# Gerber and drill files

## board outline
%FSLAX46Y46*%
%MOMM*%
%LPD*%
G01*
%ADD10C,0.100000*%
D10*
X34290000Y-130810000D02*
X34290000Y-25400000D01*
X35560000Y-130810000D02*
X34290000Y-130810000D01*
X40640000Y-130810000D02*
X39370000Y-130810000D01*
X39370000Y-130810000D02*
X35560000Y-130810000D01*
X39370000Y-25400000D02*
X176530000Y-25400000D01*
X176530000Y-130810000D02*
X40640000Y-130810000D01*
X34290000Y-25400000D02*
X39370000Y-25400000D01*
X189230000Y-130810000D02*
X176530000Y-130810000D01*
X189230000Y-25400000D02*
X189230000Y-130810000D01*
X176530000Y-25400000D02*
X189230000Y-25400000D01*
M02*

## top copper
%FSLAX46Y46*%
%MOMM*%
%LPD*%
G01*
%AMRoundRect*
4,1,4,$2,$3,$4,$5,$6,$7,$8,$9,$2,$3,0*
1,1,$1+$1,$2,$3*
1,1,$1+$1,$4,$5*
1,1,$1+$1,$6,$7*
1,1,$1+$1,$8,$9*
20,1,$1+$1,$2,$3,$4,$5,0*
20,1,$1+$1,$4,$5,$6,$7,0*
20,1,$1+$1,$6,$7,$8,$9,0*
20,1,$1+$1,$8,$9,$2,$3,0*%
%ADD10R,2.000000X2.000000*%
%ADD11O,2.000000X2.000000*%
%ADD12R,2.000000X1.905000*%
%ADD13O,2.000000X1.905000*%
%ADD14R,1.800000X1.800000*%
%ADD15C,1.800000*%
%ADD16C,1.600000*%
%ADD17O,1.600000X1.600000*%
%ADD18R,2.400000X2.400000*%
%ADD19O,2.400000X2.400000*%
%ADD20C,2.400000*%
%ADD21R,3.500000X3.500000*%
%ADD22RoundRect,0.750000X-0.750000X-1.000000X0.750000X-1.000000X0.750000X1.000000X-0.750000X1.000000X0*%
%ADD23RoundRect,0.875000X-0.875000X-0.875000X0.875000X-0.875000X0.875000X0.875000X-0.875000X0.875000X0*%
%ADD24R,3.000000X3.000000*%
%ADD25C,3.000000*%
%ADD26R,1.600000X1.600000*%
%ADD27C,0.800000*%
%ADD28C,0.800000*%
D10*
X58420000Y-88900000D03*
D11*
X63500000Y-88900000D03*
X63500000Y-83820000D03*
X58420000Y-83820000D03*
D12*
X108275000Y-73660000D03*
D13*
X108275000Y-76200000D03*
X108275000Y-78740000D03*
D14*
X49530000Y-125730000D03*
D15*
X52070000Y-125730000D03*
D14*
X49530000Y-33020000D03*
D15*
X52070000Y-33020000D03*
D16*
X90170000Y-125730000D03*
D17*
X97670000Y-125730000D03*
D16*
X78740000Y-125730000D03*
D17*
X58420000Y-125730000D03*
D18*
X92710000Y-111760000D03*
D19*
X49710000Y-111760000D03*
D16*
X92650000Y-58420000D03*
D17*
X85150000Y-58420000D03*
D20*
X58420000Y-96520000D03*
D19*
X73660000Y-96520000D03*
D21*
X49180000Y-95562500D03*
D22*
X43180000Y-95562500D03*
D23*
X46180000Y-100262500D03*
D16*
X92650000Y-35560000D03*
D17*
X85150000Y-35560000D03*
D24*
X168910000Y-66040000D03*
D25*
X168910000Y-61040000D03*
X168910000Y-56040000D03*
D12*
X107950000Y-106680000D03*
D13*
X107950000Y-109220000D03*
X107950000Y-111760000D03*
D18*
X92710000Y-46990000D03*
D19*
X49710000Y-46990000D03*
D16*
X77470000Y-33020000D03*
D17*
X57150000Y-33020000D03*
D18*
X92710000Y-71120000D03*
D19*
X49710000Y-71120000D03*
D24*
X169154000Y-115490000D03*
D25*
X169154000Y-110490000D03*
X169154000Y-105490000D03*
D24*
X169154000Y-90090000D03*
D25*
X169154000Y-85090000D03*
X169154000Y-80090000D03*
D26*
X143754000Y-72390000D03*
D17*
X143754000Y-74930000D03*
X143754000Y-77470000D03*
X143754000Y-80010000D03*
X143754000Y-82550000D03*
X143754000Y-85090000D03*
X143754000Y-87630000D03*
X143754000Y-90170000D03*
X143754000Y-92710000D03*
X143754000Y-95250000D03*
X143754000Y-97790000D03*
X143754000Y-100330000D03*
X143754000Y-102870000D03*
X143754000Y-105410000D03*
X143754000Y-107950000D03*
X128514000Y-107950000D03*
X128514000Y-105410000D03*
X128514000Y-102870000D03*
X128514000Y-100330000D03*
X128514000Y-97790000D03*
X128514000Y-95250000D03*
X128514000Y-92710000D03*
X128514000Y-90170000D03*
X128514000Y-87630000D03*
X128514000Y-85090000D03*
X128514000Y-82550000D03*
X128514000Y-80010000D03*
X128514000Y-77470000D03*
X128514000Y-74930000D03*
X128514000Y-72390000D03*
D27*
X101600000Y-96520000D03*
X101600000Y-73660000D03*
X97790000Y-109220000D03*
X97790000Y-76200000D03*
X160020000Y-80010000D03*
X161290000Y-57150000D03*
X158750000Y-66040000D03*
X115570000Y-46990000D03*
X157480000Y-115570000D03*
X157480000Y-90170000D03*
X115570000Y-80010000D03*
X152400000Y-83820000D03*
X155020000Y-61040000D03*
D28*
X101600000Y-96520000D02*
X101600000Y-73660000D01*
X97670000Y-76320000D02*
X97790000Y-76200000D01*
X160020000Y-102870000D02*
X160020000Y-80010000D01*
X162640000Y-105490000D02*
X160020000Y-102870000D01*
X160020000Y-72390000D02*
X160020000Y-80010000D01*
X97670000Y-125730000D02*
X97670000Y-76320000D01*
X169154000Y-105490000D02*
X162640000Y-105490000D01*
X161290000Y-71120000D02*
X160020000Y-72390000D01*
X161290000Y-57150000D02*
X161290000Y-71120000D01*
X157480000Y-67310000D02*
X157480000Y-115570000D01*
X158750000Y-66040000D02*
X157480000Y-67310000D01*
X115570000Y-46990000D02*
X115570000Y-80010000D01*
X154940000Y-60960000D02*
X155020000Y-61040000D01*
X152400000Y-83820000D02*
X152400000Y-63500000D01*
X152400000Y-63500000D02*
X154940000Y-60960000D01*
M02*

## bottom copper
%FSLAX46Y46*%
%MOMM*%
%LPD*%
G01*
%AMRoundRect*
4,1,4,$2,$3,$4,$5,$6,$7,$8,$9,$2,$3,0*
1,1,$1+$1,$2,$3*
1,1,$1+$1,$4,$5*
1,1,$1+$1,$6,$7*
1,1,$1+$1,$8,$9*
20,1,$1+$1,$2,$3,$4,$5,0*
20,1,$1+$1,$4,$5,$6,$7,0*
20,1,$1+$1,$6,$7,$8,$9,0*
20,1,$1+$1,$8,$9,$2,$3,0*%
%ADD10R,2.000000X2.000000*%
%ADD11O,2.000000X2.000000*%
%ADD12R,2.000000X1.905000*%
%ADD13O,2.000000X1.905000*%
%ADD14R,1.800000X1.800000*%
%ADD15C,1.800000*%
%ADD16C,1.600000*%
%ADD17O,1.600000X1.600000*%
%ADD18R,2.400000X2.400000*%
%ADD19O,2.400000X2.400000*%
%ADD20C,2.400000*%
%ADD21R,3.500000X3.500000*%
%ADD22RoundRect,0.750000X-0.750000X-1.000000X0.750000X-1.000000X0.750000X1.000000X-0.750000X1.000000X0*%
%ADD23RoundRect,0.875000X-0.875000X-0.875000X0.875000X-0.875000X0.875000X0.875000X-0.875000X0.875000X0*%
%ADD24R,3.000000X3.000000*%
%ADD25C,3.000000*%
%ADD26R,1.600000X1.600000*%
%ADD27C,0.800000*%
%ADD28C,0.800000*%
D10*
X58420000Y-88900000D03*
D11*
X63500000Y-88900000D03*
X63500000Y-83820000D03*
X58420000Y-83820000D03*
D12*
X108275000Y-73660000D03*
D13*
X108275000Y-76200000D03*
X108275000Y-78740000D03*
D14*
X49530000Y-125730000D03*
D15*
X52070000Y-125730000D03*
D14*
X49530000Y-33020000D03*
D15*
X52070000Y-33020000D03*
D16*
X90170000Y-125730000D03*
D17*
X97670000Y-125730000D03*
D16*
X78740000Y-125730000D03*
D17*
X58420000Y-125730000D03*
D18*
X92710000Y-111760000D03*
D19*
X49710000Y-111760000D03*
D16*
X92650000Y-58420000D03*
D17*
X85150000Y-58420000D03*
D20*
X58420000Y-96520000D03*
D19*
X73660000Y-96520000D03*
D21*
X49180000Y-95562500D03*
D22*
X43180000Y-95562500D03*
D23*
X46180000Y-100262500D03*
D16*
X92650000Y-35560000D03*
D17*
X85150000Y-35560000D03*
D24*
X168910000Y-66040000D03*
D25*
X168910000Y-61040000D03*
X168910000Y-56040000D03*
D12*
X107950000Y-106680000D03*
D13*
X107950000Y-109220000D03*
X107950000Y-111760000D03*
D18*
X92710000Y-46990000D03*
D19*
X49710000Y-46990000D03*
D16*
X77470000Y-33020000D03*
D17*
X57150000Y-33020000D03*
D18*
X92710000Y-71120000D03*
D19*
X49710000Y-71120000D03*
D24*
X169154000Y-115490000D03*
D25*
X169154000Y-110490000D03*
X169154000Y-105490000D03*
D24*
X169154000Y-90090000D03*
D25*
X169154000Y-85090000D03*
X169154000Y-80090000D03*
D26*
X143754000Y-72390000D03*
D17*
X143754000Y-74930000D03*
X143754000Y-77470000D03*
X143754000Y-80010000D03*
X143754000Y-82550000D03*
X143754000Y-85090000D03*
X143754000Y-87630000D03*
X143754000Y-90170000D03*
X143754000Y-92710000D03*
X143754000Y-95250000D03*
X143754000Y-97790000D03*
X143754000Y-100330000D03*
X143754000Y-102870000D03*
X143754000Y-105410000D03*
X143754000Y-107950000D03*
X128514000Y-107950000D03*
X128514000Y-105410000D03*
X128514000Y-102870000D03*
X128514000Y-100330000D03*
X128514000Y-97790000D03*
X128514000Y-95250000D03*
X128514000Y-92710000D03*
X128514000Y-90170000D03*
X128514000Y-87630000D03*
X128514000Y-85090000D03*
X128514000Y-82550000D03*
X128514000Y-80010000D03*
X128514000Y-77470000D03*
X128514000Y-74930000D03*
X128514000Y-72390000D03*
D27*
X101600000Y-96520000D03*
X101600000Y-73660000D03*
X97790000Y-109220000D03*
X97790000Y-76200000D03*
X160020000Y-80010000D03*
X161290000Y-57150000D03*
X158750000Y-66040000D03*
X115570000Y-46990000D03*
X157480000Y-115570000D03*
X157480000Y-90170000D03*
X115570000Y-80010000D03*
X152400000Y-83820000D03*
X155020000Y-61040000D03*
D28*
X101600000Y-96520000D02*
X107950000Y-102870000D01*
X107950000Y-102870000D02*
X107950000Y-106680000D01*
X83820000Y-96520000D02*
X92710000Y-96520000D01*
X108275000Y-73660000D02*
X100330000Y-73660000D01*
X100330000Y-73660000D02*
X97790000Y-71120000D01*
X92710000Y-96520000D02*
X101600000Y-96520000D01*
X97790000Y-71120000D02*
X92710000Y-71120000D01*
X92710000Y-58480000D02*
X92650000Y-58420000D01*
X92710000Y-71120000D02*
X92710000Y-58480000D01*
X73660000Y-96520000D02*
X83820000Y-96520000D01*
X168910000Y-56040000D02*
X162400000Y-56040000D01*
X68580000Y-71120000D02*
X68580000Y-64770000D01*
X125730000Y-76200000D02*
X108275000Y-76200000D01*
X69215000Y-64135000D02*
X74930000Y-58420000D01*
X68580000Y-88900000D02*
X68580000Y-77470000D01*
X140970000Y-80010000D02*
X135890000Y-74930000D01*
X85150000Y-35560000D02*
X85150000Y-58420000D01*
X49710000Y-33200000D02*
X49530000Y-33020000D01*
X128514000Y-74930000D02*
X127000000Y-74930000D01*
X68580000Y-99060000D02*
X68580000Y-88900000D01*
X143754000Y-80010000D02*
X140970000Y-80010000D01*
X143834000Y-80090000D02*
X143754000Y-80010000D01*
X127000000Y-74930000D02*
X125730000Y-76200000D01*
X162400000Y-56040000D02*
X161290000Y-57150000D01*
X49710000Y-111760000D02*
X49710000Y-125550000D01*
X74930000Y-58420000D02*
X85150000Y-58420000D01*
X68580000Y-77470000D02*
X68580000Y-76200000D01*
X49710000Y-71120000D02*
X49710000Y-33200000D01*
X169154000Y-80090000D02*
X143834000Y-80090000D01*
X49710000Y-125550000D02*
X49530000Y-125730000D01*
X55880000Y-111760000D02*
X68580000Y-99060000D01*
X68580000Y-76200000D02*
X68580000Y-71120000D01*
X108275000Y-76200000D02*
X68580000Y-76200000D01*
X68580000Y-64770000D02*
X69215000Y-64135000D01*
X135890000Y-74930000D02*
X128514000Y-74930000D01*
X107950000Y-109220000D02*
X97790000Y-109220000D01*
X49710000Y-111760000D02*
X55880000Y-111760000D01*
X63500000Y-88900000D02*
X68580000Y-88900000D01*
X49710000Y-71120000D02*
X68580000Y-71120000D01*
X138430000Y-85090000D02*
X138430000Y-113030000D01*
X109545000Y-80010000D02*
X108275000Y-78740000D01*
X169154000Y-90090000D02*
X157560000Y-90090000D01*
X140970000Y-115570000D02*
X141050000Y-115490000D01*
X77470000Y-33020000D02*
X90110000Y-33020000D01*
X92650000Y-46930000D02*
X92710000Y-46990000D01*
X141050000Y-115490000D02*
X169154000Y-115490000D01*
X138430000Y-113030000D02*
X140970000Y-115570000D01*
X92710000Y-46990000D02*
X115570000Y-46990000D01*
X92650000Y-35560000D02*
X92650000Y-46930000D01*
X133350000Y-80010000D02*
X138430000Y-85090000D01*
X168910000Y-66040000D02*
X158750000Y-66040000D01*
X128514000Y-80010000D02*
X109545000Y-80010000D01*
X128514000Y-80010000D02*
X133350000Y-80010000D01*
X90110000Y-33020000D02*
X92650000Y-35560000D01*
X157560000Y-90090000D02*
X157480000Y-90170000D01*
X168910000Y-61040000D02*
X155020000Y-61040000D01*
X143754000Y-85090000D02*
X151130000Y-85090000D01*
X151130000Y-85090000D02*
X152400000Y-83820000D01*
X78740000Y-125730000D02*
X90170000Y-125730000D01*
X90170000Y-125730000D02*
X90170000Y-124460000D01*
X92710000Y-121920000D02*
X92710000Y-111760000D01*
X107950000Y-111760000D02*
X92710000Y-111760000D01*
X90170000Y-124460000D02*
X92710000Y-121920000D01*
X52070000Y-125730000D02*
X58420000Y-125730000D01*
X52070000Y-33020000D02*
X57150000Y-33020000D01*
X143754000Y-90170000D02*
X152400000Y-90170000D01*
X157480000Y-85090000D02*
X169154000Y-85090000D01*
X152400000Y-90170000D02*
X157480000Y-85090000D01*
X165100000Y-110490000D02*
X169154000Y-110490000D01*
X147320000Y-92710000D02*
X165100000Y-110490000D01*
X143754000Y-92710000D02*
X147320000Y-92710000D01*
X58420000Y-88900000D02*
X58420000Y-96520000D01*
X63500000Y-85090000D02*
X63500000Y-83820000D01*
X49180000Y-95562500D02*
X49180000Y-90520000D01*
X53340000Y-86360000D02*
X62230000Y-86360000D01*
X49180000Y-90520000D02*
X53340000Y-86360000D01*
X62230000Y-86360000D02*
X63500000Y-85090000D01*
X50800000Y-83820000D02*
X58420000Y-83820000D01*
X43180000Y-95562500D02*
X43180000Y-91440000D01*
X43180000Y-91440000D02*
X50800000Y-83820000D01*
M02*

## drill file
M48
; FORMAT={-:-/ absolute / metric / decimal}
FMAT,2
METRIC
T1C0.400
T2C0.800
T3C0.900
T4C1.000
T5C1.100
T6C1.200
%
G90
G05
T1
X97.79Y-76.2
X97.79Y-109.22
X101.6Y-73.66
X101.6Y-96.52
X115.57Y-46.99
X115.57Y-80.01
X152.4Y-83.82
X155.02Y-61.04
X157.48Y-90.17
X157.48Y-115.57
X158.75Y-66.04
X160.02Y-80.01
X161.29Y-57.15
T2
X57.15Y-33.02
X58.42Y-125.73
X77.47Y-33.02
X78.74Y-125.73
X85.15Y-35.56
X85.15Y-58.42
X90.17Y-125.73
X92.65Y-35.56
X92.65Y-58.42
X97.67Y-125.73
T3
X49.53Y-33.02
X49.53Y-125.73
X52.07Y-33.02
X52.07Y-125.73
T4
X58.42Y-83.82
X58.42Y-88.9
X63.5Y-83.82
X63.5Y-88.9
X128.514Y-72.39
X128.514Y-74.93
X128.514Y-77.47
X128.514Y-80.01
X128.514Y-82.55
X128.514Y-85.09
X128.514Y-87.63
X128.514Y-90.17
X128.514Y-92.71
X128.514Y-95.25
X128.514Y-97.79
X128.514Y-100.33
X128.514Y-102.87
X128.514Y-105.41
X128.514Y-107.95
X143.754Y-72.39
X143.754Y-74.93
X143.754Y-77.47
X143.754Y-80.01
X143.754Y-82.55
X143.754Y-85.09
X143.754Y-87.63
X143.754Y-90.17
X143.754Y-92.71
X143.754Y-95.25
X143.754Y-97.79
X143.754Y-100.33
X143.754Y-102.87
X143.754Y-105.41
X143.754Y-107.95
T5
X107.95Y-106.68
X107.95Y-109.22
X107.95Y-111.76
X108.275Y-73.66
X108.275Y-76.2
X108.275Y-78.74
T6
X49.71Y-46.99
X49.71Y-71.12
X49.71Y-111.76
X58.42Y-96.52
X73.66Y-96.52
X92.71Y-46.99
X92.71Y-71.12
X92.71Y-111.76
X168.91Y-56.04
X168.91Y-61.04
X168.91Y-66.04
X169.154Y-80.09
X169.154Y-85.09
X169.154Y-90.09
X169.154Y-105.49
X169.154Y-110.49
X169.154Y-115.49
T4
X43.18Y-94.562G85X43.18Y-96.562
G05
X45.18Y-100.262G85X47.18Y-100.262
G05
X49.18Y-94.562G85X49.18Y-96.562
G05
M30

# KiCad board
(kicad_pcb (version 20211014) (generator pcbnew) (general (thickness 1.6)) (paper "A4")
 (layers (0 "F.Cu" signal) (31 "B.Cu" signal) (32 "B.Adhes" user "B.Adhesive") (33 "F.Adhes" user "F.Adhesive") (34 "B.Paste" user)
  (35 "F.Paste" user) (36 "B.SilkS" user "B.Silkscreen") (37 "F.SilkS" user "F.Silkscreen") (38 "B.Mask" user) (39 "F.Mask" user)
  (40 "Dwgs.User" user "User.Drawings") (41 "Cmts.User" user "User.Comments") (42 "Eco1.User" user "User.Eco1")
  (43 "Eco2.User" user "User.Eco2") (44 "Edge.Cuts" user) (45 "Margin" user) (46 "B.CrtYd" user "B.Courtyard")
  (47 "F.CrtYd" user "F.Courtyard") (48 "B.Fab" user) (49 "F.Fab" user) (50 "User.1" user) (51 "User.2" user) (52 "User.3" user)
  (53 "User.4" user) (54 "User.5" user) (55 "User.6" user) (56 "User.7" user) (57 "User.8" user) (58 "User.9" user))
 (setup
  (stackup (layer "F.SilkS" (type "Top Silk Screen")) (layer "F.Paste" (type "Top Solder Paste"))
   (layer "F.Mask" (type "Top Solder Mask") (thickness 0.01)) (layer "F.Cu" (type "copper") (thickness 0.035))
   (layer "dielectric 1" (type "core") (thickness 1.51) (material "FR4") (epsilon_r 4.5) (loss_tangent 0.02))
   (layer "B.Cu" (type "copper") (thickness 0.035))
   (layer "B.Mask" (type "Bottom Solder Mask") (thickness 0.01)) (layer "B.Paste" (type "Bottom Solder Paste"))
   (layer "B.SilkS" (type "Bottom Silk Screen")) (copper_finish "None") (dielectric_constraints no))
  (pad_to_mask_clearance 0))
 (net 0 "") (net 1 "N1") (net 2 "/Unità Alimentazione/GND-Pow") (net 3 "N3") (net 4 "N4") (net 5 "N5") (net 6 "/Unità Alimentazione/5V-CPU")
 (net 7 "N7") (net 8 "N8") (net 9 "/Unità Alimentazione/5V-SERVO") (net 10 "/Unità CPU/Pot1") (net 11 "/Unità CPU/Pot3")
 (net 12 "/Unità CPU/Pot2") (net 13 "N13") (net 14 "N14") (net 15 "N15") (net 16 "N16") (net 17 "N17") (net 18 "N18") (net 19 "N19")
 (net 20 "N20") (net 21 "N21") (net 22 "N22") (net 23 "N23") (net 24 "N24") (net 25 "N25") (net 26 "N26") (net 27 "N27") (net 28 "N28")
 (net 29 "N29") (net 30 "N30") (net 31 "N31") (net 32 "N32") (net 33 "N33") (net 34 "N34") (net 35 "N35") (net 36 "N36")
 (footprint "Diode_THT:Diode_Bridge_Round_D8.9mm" (layer "F.Cu") (at 58.42 88.9 90)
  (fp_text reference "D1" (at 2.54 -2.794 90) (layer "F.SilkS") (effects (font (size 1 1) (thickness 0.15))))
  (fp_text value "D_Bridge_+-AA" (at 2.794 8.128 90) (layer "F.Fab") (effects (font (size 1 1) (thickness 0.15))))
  (pad "1" thru_hole rect (at 0 0 90) (size 2 2) (drill 1) (layers *.Cu *.Mask) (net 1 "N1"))
  (pad "2" thru_hole oval (at 0 5.08 90) (size 2 2) (drill 1) (layers *.Cu *.Mask) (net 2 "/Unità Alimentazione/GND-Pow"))
  (pad "3" thru_hole oval (at 5.08 5.08 90) (size 2 2) (drill 1) (layers *.Cu *.Mask) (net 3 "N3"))
  (pad "4" thru_hole oval (at 5.08 0 90) (size 2 2) (drill 1) (layers *.Cu *.Mask) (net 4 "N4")))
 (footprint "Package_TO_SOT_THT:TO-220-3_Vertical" (layer "F.Cu") (at 108.275 73.66 -90)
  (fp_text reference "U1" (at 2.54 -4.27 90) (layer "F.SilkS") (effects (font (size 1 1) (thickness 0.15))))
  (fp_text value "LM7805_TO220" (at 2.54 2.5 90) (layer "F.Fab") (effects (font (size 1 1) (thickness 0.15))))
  (pad "1" thru_hole rect (at 0 0 270) (size 1.905 2) (drill 1.1) (layers *.Cu *.Mask) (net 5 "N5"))
  (pad "2" thru_hole oval (at 2.54 0 270) (size 1.905 2) (drill 1.1) (layers *.Cu *.Mask) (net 2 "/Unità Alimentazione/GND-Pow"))
  (pad "3" thru_hole oval (at 5.08 0 270) (size 1.905 2) (drill 1.1) (layers *.Cu *.Mask) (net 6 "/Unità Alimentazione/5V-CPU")))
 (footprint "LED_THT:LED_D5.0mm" (layer "F.Cu") (at 49.53 125.73)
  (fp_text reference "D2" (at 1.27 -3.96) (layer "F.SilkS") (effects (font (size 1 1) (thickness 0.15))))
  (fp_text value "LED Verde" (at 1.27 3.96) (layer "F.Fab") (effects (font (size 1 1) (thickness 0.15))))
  (pad "1" thru_hole rect (at 0 0) (size 1.8 1.8) (drill 0.9) (layers *.Cu *.Mask) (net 2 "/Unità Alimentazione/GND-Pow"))
  (pad "2" thru_hole circle (at 2.54 0) (size 1.8 1.8) (drill 0.9) (layers *.Cu *.Mask) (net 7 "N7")))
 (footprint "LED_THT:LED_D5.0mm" (layer "F.Cu") (at 49.53 33.02)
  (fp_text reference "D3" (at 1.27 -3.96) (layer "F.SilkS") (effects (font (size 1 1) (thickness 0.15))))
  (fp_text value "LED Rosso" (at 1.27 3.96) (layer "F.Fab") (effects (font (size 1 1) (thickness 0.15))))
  (pad "1" thru_hole rect (at 0 0) (size 1.8 1.8) (drill 0.9) (layers *.Cu *.Mask) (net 2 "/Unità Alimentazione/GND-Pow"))
  (pad "2" thru_hole circle (at 2.54 0) (size 1.8 1.8) (drill 0.9) (layers *.Cu *.Mask) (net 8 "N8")))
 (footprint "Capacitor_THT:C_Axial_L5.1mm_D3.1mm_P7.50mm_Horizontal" (layer "F.Cu") (at 90.17 125.73)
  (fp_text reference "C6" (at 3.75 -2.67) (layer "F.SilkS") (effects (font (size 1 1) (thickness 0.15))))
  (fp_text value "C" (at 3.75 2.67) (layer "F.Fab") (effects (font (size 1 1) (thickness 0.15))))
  (pad "1" thru_hole circle (at 0 0) (size 1.6 1.6) (drill 0.8) (layers *.Cu *.Mask) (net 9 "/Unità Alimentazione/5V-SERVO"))
  (pad "2" thru_hole oval (at 7.5 0) (size 1.6 1.6) (drill 0.8) (layers *.Cu *.Mask) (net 2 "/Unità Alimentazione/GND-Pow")))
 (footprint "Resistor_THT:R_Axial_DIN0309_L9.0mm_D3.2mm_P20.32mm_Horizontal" (layer "F.Cu") (at 78.74 125.73 180)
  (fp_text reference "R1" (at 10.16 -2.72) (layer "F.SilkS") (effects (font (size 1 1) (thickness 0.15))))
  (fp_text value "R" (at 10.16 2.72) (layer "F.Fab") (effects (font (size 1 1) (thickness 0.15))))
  (pad "1" thru_hole circle (at 0 0 180) (size 1.6 1.6) (drill 0.8) (layers *.Cu *.Mask) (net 9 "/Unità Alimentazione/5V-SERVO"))
  (pad "2" thru_hole oval (at 20.32 0 180) (size 1.6 1.6) (drill 0.8) (layers *.Cu *.Mask) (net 7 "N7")))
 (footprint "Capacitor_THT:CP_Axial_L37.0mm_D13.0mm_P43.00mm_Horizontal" (layer "F.Cu") (at 92.71 111.76 180)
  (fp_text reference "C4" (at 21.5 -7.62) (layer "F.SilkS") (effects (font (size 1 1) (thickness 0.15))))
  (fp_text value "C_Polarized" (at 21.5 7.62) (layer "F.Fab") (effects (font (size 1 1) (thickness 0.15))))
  (pad "1" thru_hole rect (at 0 0 180) (size 2.4 2.4) (drill 1.2) (layers *.Cu *.Mask) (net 9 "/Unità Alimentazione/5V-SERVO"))
  (pad "2" thru_hole oval (at 43 0 180) (size 2.4 2.4) (drill 1.2) (layers *.Cu *.Mask) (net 2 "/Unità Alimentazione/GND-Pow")))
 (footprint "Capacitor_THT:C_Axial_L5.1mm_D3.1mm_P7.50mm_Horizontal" (layer "F.Cu") (at 92.65 58.42 180)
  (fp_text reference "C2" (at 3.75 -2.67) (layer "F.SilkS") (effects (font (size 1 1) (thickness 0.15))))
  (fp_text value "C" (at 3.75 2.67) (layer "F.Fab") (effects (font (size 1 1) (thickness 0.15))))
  (pad "1" thru_hole circle (at 0 0 180) (size 1.6 1.6) (drill 0.8) (layers *.Cu *.Mask) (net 5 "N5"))
  (pad "2" thru_hole oval (at 7.5 0 180) (size 1.6 1.6) (drill 0.8) (layers *.Cu *.Mask) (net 2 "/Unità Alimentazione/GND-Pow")))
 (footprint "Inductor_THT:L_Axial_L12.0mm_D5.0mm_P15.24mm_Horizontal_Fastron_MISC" (layer "F.Cu") (at 58.42 96.52)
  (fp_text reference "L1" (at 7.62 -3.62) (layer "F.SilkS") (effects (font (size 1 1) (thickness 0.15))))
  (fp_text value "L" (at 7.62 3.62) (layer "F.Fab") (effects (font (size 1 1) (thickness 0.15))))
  (pad "1" thru_hole circle (at 0 0) (size 2.4 2.4) (drill 1.2) (layers *.Cu *.Mask) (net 1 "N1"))
  (pad "2" thru_hole oval (at 15.24 0) (size 2.4 2.4) (drill 1.2) (layers *.Cu *.Mask) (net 5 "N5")))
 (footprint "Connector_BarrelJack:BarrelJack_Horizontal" (layer "F.Cu") (at 49.18 95.5625)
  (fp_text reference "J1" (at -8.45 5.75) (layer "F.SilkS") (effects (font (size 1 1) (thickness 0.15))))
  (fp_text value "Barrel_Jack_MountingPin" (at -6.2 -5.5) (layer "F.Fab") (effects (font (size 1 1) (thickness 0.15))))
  (pad "1" thru_hole rect (at 0 0) (size 3.5 3.5) (drill oval 1 3) (layers *.Cu *.Mask) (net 3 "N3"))
  (pad "2" thru_hole roundrect (at -6 0) (size 3 3.5) (drill oval 1 3) (layers *.Cu *.Mask) (roundrect_rratio 0.25) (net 4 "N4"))
  (pad "3" thru_hole roundrect (at -3 4.7) (size 3.5 3.5) (drill oval 3 1) (layers *.Cu *.Mask) (roundrect_rratio 0.25)))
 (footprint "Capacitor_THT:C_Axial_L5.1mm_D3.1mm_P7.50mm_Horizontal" (layer "F.Cu") (at 92.65 35.56 180)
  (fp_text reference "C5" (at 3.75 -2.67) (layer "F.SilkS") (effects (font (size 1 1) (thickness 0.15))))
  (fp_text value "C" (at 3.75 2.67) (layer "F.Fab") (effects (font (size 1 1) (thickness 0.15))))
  (pad "1" thru_hole circle (at 0 0 180) (size 1.6 1.6) (drill 0.8) (layers *.Cu *.Mask) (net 6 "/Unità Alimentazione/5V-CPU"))
  (pad "2" thru_hole oval (at 7.5 0 180) (size 1.6 1.6) (drill 0.8) (layers *.Cu *.Mask) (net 2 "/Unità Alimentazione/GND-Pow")))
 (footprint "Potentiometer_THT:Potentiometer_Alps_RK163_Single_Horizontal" (layer "F.Cu") (at 168.91 66.04 180)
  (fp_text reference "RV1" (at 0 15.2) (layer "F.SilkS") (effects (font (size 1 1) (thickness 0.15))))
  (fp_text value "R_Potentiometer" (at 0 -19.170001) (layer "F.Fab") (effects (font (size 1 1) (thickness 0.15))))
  (pad "1" thru_hole rect (at 0 0) (size 3 3) (drill 1.2) (layers *.Cu *.Mask) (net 6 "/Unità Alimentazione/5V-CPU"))
  (pad "2" thru_hole circle (at 0 5) (size 3 3) (drill 1.2) (layers *.Cu *.Mask) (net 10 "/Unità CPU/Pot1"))
  (pad "3" thru_hole circle (at 0 10) (size 3 3) (drill 1.2) (layers *.Cu *.Mask) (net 2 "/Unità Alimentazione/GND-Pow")))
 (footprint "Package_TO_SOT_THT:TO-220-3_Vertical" (layer "F.Cu") (at 107.95 106.68 -90)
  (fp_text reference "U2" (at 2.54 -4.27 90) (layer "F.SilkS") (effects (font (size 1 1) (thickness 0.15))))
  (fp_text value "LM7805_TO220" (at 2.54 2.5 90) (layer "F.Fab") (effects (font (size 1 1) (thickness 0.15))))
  (pad "1" thru_hole rect (at 0 0 270) (size 1.905 2) (drill 1.1) (layers *.Cu *.Mask) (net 5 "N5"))
  (pad "2" thru_hole oval (at 2.54 0 270) (size 1.905 2) (drill 1.1) (layers *.Cu *.Mask) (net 2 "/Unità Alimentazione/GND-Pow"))
  (pad "3" thru_hole oval (at 5.08 0 270) (size 1.905 2) (drill 1.1) (layers *.Cu *.Mask) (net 9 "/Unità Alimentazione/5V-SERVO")))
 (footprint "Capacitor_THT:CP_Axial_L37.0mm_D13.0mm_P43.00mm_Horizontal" (layer "F.Cu") (at 92.71 46.99 180)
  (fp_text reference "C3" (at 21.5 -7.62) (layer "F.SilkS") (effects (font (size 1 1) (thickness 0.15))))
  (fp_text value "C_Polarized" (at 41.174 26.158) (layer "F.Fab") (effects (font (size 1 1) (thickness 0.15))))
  (pad "1" thru_hole rect (at 0 0 180) (size 2.4 2.4) (drill 1.2) (layers *.Cu *.Mask) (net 6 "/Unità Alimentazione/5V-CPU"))
  (pad "2" thru_hole oval (at 43 0 180) (size 2.4 2.4) (drill 1.2) (layers *.Cu *.Mask) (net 2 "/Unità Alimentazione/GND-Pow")))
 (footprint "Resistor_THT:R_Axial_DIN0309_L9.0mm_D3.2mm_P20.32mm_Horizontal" (layer "F.Cu") (at 77.47 33.02 180)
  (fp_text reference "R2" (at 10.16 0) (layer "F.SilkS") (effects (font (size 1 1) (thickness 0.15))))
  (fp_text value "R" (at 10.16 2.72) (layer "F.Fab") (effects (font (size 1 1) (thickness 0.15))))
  (pad "1" thru_hole circle (at 0 0 180) (size 1.6 1.6) (drill 0.8) (layers *.Cu *.Mask) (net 6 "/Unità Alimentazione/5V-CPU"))
  (pad "2" thru_hole oval (at 20.32 0 180) (size 1.6 1.6) (drill 0.8) (layers *.Cu *.Mask) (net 8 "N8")))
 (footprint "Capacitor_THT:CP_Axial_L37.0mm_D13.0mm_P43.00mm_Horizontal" (layer "F.Cu") (at 92.71 71.12 180)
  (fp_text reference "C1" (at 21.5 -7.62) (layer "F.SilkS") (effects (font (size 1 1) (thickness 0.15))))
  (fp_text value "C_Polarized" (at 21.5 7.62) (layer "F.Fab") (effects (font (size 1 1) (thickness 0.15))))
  (pad "1" thru_hole rect (at 0 0 180) (size 2.4 2.4) (drill 1.2) (layers *.Cu *.Mask) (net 5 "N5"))
  (pad "2" thru_hole oval (at 43 0 180) (size 2.4 2.4) (drill 1.2) (layers *.Cu *.Mask) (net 2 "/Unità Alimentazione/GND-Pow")))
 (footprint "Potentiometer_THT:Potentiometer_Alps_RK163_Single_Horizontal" (layer "F.Cu") (at 169.154 115.49 180)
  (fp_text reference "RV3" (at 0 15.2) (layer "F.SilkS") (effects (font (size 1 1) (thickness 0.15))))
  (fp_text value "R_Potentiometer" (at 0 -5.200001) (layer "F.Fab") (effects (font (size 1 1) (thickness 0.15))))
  (pad "1" thru_hole rect (at 0 0) (size 3 3) (drill 1.2) (layers *.Cu *.Mask) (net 6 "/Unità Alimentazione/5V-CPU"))
  (pad "2" thru_hole circle (at 0 5) (size 3 3) (drill 1.2) (layers *.Cu *.Mask) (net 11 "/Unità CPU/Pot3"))
  (pad "3" thru_hole circle (at 0 10) (size 3 3) (drill 1.2) (layers *.Cu *.Mask) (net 2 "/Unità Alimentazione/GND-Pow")))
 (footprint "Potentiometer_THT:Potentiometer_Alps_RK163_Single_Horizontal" (layer "F.Cu") (at 169.154 90.09 180)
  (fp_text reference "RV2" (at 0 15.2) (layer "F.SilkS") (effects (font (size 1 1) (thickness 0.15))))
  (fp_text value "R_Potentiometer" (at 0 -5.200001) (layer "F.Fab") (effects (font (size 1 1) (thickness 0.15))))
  (pad "1" thru_hole rect (at 0 0) (size 3 3) (drill 1.2) (layers *.Cu *.Mask) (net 6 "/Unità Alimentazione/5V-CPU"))
  (pad "2" thru_hole circle (at 0 5) (size 3 3) (drill 1.2) (layers *.Cu *.Mask) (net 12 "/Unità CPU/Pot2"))
  (pad "3" thru_hole circle (at 0 10) (size 3 3) (drill 1.2) (layers *.Cu *.Mask) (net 2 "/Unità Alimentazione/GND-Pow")))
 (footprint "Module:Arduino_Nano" (layer "B.Cu") (at 143.754 72.39 180)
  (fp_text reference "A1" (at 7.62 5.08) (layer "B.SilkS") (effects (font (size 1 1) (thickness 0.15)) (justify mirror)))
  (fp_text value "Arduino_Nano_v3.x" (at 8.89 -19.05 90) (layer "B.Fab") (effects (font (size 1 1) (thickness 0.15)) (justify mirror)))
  (pad "1" thru_hole rect (at 0 0 180) (size 1.6 1.6) (drill 1) (layers *.Cu *.Mask) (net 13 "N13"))
  (pad "2" thru_hole oval (at 0 -2.54 180) (size 1.6 1.6) (drill 1) (layers *.Cu *.Mask) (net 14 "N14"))
  (pad "3" thru_hole oval (at 0 -5.08 180) (size 1.6 1.6) (drill 1) (layers *.Cu *.Mask) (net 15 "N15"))
  (pad "4" thru_hole oval (at 0 -7.62 180) (size 1.6 1.6) (drill 1) (layers *.Cu *.Mask) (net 2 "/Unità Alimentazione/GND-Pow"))
  (pad "5" thru_hole oval (at 0 -10.16 180) (size 1.6 1.6) (drill 1) (layers *.Cu *.Mask) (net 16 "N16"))
  (pad "6" thru_hole oval (at 0 -12.7 180) (size 1.6 1.6) (drill 1) (layers *.Cu *.Mask) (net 10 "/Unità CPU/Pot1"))
  (pad "7" thru_hole oval (at 0 -15.24 180) (size 1.6 1.6) (drill 1) (layers *.Cu *.Mask) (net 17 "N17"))
  (pad "8" thru_hole oval (at 0 -17.78 180) (size 1.6 1.6) (drill 1) (layers *.Cu *.Mask) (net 12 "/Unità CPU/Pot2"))
  (pad "9" thru_hole oval (at 0 -20.32 180) (size 1.6 1.6) (drill 1) (layers *.Cu *.Mask) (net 11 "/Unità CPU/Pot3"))
  (pad "10" thru_hole oval (at 0 -22.86 180) (size 1.6 1.6) (drill 1) (layers *.Cu *.Mask) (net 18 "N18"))
  (pad "11" thru_hole oval (at 0 -25.4 180) (size 1.6 1.6) (drill 1) (layers *.Cu *.Mask) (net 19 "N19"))
  (pad "12" thru_hole oval (at 0 -27.94 180) (size 1.6 1.6) (drill 1) (layers *.Cu *.Mask) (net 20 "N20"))
  (pad "13" thru_hole oval (at 0 -30.48 180) (size 1.6 1.6) (drill 1) (layers *.Cu *.Mask) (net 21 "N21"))
  (pad "14" thru_hole oval (at 0 -33.02 180) (size 1.6 1.6) (drill 1) (layers *.Cu *.Mask) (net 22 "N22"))
  (pad "15" thru_hole oval (at 0 -35.56 180) (size 1.6 1.6) (drill 1) (layers *.Cu *.Mask) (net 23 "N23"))
  (pad "16" thru_hole oval (at 15.24 -35.56 180) (size 1.6 1.6) (drill 1) (layers *.Cu *.Mask) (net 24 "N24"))
  (pad "17" thru_hole oval (at 15.24 -33.02 180) (size 1.6 1.6) (drill 1) (layers *.Cu *.Mask) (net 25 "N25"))
  (pad "18" thru_hole oval (at 15.24 -30.48 180) (size 1.6 1.6) (drill 1) (layers *.Cu *.Mask) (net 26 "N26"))
  (pad "19" thru_hole oval (at 15.24 -27.94 180) (size 1.6 1.6) (drill 1) (layers *.Cu *.Mask) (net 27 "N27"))
  (pad "20" thru_hole oval (at 15.24 -25.4 180) (size 1.6 1.6) (drill 1) (layers *.Cu *.Mask) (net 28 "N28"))
  (pad "21" thru_hole oval (at 15.24 -22.86 180) (size 1.6 1.6) (drill 1) (layers *.Cu *.Mask) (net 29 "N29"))
  (pad "22" thru_hole oval (at 15.24 -20.32 180) (size 1.6 1.6) (drill 1) (layers *.Cu *.Mask) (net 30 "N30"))
  (pad "23" thru_hole oval (at 15.24 -17.78 180) (size 1.6 1.6) (drill 1) (layers *.Cu *.Mask) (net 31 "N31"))
  (pad "24" thru_hole oval (at 15.24 -15.24 180) (size 1.6 1.6) (drill 1) (layers *.Cu *.Mask) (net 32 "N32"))
  (pad "25" thru_hole oval (at 15.24 -12.7 180) (size 1.6 1.6) (drill 1) (layers *.Cu *.Mask) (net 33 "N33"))
  (pad "26" thru_hole oval (at 15.24 -10.16 180) (size 1.6 1.6) (drill 1) (layers *.Cu *.Mask) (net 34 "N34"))
  (pad "27" thru_hole oval (at 15.24 -7.62 180) (size 1.6 1.6) (drill 1) (layers *.Cu *.Mask) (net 6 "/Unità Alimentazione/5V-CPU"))
  (pad "28" thru_hole oval (at 15.24 -5.08 180) (size 1.6 1.6) (drill 1) (layers *.Cu *.Mask) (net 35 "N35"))
  (pad "29" thru_hole oval (at 15.24 -2.54 180) (size 1.6 1.6) (drill 1) (layers *.Cu *.Mask) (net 2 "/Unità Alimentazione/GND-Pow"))
  (pad "30" thru_hole oval (at 15.24 0 180) (size 1.6 1.6) (drill 1) (layers *.Cu *.Mask) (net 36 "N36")))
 (gr_line (start 34.29 130.81) (end 34.29 25.4) (layer "Edge.Cuts") (width 0.1))
 (gr_line (start 35.56 130.81) (end 34.29 130.81) (layer "Edge.Cuts") (width 0.1))
 (gr_line (start 40.64 130.81) (end 39.37 130.81) (layer "Edge.Cuts") (width 0.1))
 (gr_line (start 39.37 130.81) (end 35.56 130.81) (layer "Edge.Cuts") (width 0.1))
 (gr_line (start 39.37 25.4) (end 176.53 25.4) (layer "Edge.Cuts") (width 0.1))
 (gr_line (start 176.53 130.81) (end 40.64 130.81) (layer "Edge.Cuts") (width 0.1))
 (gr_line (start 34.29 25.4) (end 39.37 25.4) (layer "Edge.Cuts") (width 0.1))
 (gr_line (start 189.23 130.81) (end 176.53 130.81) (layer "Edge.Cuts") (width 0.1))
 (gr_line (start 189.23 25.4) (end 189.23 130.81) (layer "Edge.Cuts") (width 0.1))
 (gr_line (start 176.53 25.4) (end 189.23 25.4) (layer "Edge.Cuts") (width 0.1))
 (segment (start 101.6 96.52) (end 101.6 73.66) (width 0.8) (layer "F.Cu") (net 5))
 (via (at 101.6 96.52) (size 0.8) (drill 0.4) (layers "F.Cu" "B.Cu") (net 5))
 (via (at 101.6 73.66) (size 0.8) (drill 0.4) (layers "F.Cu" "B.Cu") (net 5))
 (segment (start 101.6 96.52) (end 107.95 102.87) (width 0.8) (layer "B.Cu") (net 5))
 (segment (start 107.95 102.87) (end 107.95 106.68) (width 0.8) (layer "B.Cu") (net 5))
 (segment (start 83.82 96.52) (end 92.71 96.52) (width 0.8) (layer "B.Cu") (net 5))
 (segment (start 108.275 73.66) (end 100.33 73.66) (width 0.8) (layer "B.Cu") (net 5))
 (segment (start 100.33 73.66) (end 97.79 71.12) (width 0.8) (layer "B.Cu") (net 5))
 (segment (start 92.71 96.52) (end 101.6 96.52) (width 0.8) (layer "B.Cu") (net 5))
 (segment (start 97.79 71.12) (end 92.71 71.12) (width 0.8) (layer "B.Cu") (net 5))
 (segment (start 92.71 58.48) (end 92.65 58.42) (width 0.8) (layer "B.Cu") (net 5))
 (segment (start 92.71 71.12) (end 92.71 58.48) (width 0.8) (layer "B.Cu") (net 5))
 (segment (start 73.66 96.52) (end 83.82 96.52) (width 0.8) (layer "B.Cu") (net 5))
 (segment (start 97.67 76.32) (end 97.79 76.2) (width 0.8) (layer "F.Cu") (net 2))
 (segment (start 160.02 102.87) (end 160.02 80.01) (width 0.8) (layer "F.Cu") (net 2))
 (segment (start 162.64 105.49) (end 160.02 102.87) (width 0.8) (layer "F.Cu") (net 2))
 (segment (start 160.02 72.39) (end 160.02 80.01) (width 0.8) (layer "F.Cu") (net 2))
 (segment (start 97.67 125.73) (end 97.67 76.32) (width 0.8) (layer "F.Cu") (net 2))
 (segment (start 169.154 105.49) (end 162.64 105.49) (width 0.8) (layer "F.Cu") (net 2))
 (segment (start 161.29 71.12) (end 160.02 72.39) (width 0.8) (layer "F.Cu") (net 2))
 (segment (start 161.29 57.15) (end 161.29 71.12) (width 0.8) (layer "F.Cu") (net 2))
 (via (at 97.79 109.22) (size 0.8) (drill 0.4) (layers "F.Cu" "B.Cu") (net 2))
 (via (at 97.79 76.2) (size 0.8) (drill 0.4) (layers "F.Cu" "B.Cu") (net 2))
 (via (at 160.02 80.01) (size 0.8) (drill 0.4) (layers "F.Cu" "B.Cu") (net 2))
 (via (at 161.29 57.15) (size 0.8) (drill 0.4) (layers "F.Cu" "B.Cu") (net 2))
 (segment (start 168.91 56.04) (end 162.4 56.04) (width 0.8) (layer "B.Cu") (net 2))
 (segment (start 68.58 71.12) (end 68.58 64.77) (width 0.8) (layer "B.Cu") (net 2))
 (segment (start 125.73 76.2) (end 108.275 76.2) (width 0.8) (layer "B.Cu") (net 2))
 (segment (start 69.215 64.135) (end 74.93 58.42) (width 0.8) (layer "B.Cu") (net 2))
 (segment (start 68.58 88.9) (end 68.58 77.47) (width 0.8) (layer "B.Cu") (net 2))
 (segment (start 140.97 80.01) (end 135.89 74.93) (width 0.8) (layer "B.Cu") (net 2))
 (segment (start 85.15 35.56) (end 85.15 58.42) (width 0.8) (layer "B.Cu") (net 2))
 (segment (start 49.71 33.2) (end 49.53 33.02) (width 0.8) (layer "B.Cu") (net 2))
 (segment (start 128.514 74.93) (end 127 74.93) (width 0.8) (layer "B.Cu") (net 2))
 (segment (start 68.58 99.06) (end 68.58 88.9) (width 0.8) (layer "B.Cu") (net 2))
 (segment (start 143.754 80.01) (end 140.97 80.01) (width 0.8) (layer "B.Cu") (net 2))
 (segment (start 143.834 80.09) (end 143.754 80.01) (width 0.8) (layer "B.Cu") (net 2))
 (segment (start 127 74.93) (end 125.73 76.2) (width 0.8) (layer "B.Cu") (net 2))
 (segment (start 162.4 56.04) (end 161.29 57.15) (width 0.8) (layer "B.Cu") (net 2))
 (segment (start 49.71 111.76) (end 49.71 125.55) (width 0.8) (layer "B.Cu") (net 2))
 (segment (start 74.93 58.42) (end 85.15 58.42) (width 0.8) (layer "B.Cu") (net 2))
 (segment (start 68.58 77.47) (end 68.58 76.2) (width 0.8) (layer "B.Cu") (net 2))
 (segment (start 49.71 71.12) (end 49.71 33.2) (width 0.8) (layer "B.Cu") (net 2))
 (segment (start 169.154 80.09) (end 143.834 80.09) (width 0.8) (layer "B.Cu") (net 2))
 (segment (start 49.71 125.55) (end 49.53 125.73) (width 0.8) (layer "B.Cu") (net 2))
 (segment (start 55.88 111.76) (end 68.58 99.06) (width 0.8) (layer "B.Cu") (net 2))
 (segment (start 68.58 76.2) (end 68.58 71.12) (width 0.8) (layer "B.Cu") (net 2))
 (segment (start 108.275 76.2) (end 68.58 76.2) (width 0.8) (layer "B.Cu") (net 2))
 (segment (start 68.58 64.77) (end 69.215 64.135) (width 0.8) (layer "B.Cu") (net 2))
 (segment (start 135.89 74.93) (end 128.514 74.93) (width 0.8) (layer "B.Cu") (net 2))
 (segment (start 107.95 109.22) (end 97.79 109.22) (width 0.8) (layer "B.Cu") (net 2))
 (segment (start 49.71 111.76) (end 55.88 111.76) (width 0.8) (layer "B.Cu") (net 2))
 (segment (start 63.5 88.9) (end 68.58 88.9) (width 0.8) (layer "B.Cu") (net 2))
 (segment (start 49.71 71.12) (end 68.58 71.12) (width 0.8) (layer "B.Cu") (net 2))
 (segment (start 157.48 67.31) (end 157.48 115.57) (width 0.8) (layer "F.Cu") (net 6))
 (segment (start 158.75 66.04) (end 157.48 67.31) (width 0.8) (layer "F.Cu") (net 6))
 (segment (start 115.57 46.99) (end 115.57 80.01) (width 0.8) (layer "F.Cu") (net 6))
 (via (at 158.75 66.04) (size 0.8) (drill 0.4) (layers "F.Cu" "B.Cu") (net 6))
 (via (at 115.57 46.99) (size 0.8) (drill 0.4) (layers "F.Cu" "B.Cu") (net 6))
 (via (at 157.48 115.57) (size 0.8) (drill 0.4) (layers "F.Cu" "B.Cu") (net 6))
 (via (at 157.48 90.17) (size 0.8) (drill 0.4) (layers "F.Cu" "B.Cu") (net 6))
 (via (at 115.57 80.01) (size 0.8) (drill 0.4) (layers "F.Cu" "B.Cu") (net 6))
 (segment (start 138.43 85.09) (end 138.43 113.03) (width 0.8) (layer "B.Cu") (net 6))
 (segment (start 109.545 80.01) (end 108.275 78.74) (width 0.8) (layer "B.Cu") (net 6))
 (segment (start 169.154 90.09) (end 157.56 90.09) (width 0.8) (layer "B.Cu") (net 6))
 (segment (start 140.97 115.57) (end 141.05 115.49) (width 0.8) (layer "B.Cu") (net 6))
 (segment (start 77.47 33.02) (end 90.11 33.02) (width 0.8) (layer "B.Cu") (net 6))
 (segment (start 92.65 46.93) (end 92.71 46.99) (width 0.8) (layer "B.Cu") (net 6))
 (segment (start 141.05 115.49) (end 169.154 115.49) (width 0.8) (layer "B.Cu") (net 6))
 (segment (start 138.43 113.03) (end 140.97 115.57) (width 0.8) (layer "B.Cu") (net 6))
 (segment (start 92.71 46.99) (end 115.57 46.99) (width 0.8) (layer "B.Cu") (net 6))
 (segment (start 92.65 35.56) (end 92.65 46.93) (width 0.8) (layer "B.Cu") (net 6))
 (segment (start 133.35 80.01) (end 138.43 85.09) (width 0.8) (layer "B.Cu") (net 6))
 (segment (start 168.91 66.04) (end 158.75 66.04) (width 0.8) (layer "B.Cu") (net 6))
 (segment (start 128.514 80.01) (end 109.545 80.01) (width 0.8) (layer "B.Cu") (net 6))
 (segment (start 128.514 80.01) (end 133.35 80.01) (width 0.8) (layer "B.Cu") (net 6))
 (segment (start 90.11 33.02) (end 92.65 35.56) (width 0.8) (layer "B.Cu") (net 6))
 (segment (start 157.56 90.09) (end 157.48 90.17) (width 0.8) (layer "B.Cu") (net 6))
 (segment (start 154.94 60.96) (end 155.02 61.04) (width 0.8) (layer "F.Cu") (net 10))
 (segment (start 152.4 83.82) (end 152.4 63.5) (width 0.8) (layer "F.Cu") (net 10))
 (segment (start 152.4 63.5) (end 154.94 60.96) (width 0.8) (layer "F.Cu") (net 10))
 (via (at 152.4 83.82) (size 0.8) (drill 0.4) (layers "F.Cu" "B.Cu") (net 10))
 (via (at 155.02 61.04) (size 0.8) (drill 0.4) (layers "F.Cu" "B.Cu") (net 10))
 (segment (start 168.91 61.04) (end 155.02 61.04) (width 0.8) (layer "B.Cu") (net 10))
 (segment (start 143.754 85.09) (end 151.13 85.09) (width 0.8) (layer "B.Cu") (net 10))
 (segment (start 151.13 85.09) (end 152.4 83.82) (width 0.8) (layer "B.Cu") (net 10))
 (segment (start 78.74 125.73) (end 90.17 125.73) (width 0.8) (layer "B.Cu") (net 9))
 (segment (start 90.17 125.73) (end 90.17 124.46) (width 0.8) (layer "B.Cu") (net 9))
 (segment (start 92.71 121.92) (end 92.71 111.76) (width 0.8) (layer "B.Cu") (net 9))
 (segment (start 107.95 111.76) (end 92.71 111.76) (width 0.8) (layer "B.Cu") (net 9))
 (segment (start 90.17 124.46) (end 92.71 121.92) (width 0.8) (layer "B.Cu") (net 9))
 (segment (start 52.07 125.73) (end 58.42 125.73) (width 0.8) (layer "B.Cu") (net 7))
 (segment (start 52.07 33.02) (end 57.15 33.02) (width 0.8) (layer "B.Cu") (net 8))
 (segment (start 143.754 90.17) (end 152.4 90.17) (width 0.8) (layer "B.Cu") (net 12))
 (segment (start 157.48 85.09) (end 169.154 85.09) (width 0.8) (layer "B.Cu") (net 12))
 (segment (start 152.4 90.17) (end 157.48 85.09) (width 0.8) (layer "B.Cu") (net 12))
 (segment (start 165.1 110.49) (end 169.154 110.49) (width 0.8) (layer "B.Cu") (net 11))
 (segment (start 147.32 92.71) (end 165.1 110.49) (width 0.8) (layer "B.Cu") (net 11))
 (segment (start 143.754 92.71) (end 147.32 92.71) (width 0.8) (layer "B.Cu") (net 11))
 (segment (start 58.42 88.9) (end 58.42 96.52) (width 0.8) (layer "B.Cu") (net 1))
 (segment (start 63.5 85.09) (end 63.5 83.82) (width 0.8) (layer "B.Cu") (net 3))
 (segment (start 49.18 95.5625) (end 49.18 90.52) (width 0.8) (layer "B.Cu") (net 3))
 (segment (start 53.34 86.36) (end 62.23 86.36) (width 0.8) (layer "B.Cu") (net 3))
 (segment (start 49.18 90.52) (end 53.34 86.36) (width 0.8) (layer "B.Cu") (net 3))
 (segment (start 62.23 86.36) (end 63.5 85.09) (width 0.8) (layer "B.Cu") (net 3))
 (segment (start 50.8 83.82) (end 58.42 83.82) (width 0.8) (layer "B.Cu") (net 4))
 (segment (start 43.18 95.5625) (end 43.18 91.44) (width 0.8) (layer "B.Cu") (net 4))
 (segment (start 43.18 91.44) (end 50.8 83.82) (width 0.8) (layer "B.Cu") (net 4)))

